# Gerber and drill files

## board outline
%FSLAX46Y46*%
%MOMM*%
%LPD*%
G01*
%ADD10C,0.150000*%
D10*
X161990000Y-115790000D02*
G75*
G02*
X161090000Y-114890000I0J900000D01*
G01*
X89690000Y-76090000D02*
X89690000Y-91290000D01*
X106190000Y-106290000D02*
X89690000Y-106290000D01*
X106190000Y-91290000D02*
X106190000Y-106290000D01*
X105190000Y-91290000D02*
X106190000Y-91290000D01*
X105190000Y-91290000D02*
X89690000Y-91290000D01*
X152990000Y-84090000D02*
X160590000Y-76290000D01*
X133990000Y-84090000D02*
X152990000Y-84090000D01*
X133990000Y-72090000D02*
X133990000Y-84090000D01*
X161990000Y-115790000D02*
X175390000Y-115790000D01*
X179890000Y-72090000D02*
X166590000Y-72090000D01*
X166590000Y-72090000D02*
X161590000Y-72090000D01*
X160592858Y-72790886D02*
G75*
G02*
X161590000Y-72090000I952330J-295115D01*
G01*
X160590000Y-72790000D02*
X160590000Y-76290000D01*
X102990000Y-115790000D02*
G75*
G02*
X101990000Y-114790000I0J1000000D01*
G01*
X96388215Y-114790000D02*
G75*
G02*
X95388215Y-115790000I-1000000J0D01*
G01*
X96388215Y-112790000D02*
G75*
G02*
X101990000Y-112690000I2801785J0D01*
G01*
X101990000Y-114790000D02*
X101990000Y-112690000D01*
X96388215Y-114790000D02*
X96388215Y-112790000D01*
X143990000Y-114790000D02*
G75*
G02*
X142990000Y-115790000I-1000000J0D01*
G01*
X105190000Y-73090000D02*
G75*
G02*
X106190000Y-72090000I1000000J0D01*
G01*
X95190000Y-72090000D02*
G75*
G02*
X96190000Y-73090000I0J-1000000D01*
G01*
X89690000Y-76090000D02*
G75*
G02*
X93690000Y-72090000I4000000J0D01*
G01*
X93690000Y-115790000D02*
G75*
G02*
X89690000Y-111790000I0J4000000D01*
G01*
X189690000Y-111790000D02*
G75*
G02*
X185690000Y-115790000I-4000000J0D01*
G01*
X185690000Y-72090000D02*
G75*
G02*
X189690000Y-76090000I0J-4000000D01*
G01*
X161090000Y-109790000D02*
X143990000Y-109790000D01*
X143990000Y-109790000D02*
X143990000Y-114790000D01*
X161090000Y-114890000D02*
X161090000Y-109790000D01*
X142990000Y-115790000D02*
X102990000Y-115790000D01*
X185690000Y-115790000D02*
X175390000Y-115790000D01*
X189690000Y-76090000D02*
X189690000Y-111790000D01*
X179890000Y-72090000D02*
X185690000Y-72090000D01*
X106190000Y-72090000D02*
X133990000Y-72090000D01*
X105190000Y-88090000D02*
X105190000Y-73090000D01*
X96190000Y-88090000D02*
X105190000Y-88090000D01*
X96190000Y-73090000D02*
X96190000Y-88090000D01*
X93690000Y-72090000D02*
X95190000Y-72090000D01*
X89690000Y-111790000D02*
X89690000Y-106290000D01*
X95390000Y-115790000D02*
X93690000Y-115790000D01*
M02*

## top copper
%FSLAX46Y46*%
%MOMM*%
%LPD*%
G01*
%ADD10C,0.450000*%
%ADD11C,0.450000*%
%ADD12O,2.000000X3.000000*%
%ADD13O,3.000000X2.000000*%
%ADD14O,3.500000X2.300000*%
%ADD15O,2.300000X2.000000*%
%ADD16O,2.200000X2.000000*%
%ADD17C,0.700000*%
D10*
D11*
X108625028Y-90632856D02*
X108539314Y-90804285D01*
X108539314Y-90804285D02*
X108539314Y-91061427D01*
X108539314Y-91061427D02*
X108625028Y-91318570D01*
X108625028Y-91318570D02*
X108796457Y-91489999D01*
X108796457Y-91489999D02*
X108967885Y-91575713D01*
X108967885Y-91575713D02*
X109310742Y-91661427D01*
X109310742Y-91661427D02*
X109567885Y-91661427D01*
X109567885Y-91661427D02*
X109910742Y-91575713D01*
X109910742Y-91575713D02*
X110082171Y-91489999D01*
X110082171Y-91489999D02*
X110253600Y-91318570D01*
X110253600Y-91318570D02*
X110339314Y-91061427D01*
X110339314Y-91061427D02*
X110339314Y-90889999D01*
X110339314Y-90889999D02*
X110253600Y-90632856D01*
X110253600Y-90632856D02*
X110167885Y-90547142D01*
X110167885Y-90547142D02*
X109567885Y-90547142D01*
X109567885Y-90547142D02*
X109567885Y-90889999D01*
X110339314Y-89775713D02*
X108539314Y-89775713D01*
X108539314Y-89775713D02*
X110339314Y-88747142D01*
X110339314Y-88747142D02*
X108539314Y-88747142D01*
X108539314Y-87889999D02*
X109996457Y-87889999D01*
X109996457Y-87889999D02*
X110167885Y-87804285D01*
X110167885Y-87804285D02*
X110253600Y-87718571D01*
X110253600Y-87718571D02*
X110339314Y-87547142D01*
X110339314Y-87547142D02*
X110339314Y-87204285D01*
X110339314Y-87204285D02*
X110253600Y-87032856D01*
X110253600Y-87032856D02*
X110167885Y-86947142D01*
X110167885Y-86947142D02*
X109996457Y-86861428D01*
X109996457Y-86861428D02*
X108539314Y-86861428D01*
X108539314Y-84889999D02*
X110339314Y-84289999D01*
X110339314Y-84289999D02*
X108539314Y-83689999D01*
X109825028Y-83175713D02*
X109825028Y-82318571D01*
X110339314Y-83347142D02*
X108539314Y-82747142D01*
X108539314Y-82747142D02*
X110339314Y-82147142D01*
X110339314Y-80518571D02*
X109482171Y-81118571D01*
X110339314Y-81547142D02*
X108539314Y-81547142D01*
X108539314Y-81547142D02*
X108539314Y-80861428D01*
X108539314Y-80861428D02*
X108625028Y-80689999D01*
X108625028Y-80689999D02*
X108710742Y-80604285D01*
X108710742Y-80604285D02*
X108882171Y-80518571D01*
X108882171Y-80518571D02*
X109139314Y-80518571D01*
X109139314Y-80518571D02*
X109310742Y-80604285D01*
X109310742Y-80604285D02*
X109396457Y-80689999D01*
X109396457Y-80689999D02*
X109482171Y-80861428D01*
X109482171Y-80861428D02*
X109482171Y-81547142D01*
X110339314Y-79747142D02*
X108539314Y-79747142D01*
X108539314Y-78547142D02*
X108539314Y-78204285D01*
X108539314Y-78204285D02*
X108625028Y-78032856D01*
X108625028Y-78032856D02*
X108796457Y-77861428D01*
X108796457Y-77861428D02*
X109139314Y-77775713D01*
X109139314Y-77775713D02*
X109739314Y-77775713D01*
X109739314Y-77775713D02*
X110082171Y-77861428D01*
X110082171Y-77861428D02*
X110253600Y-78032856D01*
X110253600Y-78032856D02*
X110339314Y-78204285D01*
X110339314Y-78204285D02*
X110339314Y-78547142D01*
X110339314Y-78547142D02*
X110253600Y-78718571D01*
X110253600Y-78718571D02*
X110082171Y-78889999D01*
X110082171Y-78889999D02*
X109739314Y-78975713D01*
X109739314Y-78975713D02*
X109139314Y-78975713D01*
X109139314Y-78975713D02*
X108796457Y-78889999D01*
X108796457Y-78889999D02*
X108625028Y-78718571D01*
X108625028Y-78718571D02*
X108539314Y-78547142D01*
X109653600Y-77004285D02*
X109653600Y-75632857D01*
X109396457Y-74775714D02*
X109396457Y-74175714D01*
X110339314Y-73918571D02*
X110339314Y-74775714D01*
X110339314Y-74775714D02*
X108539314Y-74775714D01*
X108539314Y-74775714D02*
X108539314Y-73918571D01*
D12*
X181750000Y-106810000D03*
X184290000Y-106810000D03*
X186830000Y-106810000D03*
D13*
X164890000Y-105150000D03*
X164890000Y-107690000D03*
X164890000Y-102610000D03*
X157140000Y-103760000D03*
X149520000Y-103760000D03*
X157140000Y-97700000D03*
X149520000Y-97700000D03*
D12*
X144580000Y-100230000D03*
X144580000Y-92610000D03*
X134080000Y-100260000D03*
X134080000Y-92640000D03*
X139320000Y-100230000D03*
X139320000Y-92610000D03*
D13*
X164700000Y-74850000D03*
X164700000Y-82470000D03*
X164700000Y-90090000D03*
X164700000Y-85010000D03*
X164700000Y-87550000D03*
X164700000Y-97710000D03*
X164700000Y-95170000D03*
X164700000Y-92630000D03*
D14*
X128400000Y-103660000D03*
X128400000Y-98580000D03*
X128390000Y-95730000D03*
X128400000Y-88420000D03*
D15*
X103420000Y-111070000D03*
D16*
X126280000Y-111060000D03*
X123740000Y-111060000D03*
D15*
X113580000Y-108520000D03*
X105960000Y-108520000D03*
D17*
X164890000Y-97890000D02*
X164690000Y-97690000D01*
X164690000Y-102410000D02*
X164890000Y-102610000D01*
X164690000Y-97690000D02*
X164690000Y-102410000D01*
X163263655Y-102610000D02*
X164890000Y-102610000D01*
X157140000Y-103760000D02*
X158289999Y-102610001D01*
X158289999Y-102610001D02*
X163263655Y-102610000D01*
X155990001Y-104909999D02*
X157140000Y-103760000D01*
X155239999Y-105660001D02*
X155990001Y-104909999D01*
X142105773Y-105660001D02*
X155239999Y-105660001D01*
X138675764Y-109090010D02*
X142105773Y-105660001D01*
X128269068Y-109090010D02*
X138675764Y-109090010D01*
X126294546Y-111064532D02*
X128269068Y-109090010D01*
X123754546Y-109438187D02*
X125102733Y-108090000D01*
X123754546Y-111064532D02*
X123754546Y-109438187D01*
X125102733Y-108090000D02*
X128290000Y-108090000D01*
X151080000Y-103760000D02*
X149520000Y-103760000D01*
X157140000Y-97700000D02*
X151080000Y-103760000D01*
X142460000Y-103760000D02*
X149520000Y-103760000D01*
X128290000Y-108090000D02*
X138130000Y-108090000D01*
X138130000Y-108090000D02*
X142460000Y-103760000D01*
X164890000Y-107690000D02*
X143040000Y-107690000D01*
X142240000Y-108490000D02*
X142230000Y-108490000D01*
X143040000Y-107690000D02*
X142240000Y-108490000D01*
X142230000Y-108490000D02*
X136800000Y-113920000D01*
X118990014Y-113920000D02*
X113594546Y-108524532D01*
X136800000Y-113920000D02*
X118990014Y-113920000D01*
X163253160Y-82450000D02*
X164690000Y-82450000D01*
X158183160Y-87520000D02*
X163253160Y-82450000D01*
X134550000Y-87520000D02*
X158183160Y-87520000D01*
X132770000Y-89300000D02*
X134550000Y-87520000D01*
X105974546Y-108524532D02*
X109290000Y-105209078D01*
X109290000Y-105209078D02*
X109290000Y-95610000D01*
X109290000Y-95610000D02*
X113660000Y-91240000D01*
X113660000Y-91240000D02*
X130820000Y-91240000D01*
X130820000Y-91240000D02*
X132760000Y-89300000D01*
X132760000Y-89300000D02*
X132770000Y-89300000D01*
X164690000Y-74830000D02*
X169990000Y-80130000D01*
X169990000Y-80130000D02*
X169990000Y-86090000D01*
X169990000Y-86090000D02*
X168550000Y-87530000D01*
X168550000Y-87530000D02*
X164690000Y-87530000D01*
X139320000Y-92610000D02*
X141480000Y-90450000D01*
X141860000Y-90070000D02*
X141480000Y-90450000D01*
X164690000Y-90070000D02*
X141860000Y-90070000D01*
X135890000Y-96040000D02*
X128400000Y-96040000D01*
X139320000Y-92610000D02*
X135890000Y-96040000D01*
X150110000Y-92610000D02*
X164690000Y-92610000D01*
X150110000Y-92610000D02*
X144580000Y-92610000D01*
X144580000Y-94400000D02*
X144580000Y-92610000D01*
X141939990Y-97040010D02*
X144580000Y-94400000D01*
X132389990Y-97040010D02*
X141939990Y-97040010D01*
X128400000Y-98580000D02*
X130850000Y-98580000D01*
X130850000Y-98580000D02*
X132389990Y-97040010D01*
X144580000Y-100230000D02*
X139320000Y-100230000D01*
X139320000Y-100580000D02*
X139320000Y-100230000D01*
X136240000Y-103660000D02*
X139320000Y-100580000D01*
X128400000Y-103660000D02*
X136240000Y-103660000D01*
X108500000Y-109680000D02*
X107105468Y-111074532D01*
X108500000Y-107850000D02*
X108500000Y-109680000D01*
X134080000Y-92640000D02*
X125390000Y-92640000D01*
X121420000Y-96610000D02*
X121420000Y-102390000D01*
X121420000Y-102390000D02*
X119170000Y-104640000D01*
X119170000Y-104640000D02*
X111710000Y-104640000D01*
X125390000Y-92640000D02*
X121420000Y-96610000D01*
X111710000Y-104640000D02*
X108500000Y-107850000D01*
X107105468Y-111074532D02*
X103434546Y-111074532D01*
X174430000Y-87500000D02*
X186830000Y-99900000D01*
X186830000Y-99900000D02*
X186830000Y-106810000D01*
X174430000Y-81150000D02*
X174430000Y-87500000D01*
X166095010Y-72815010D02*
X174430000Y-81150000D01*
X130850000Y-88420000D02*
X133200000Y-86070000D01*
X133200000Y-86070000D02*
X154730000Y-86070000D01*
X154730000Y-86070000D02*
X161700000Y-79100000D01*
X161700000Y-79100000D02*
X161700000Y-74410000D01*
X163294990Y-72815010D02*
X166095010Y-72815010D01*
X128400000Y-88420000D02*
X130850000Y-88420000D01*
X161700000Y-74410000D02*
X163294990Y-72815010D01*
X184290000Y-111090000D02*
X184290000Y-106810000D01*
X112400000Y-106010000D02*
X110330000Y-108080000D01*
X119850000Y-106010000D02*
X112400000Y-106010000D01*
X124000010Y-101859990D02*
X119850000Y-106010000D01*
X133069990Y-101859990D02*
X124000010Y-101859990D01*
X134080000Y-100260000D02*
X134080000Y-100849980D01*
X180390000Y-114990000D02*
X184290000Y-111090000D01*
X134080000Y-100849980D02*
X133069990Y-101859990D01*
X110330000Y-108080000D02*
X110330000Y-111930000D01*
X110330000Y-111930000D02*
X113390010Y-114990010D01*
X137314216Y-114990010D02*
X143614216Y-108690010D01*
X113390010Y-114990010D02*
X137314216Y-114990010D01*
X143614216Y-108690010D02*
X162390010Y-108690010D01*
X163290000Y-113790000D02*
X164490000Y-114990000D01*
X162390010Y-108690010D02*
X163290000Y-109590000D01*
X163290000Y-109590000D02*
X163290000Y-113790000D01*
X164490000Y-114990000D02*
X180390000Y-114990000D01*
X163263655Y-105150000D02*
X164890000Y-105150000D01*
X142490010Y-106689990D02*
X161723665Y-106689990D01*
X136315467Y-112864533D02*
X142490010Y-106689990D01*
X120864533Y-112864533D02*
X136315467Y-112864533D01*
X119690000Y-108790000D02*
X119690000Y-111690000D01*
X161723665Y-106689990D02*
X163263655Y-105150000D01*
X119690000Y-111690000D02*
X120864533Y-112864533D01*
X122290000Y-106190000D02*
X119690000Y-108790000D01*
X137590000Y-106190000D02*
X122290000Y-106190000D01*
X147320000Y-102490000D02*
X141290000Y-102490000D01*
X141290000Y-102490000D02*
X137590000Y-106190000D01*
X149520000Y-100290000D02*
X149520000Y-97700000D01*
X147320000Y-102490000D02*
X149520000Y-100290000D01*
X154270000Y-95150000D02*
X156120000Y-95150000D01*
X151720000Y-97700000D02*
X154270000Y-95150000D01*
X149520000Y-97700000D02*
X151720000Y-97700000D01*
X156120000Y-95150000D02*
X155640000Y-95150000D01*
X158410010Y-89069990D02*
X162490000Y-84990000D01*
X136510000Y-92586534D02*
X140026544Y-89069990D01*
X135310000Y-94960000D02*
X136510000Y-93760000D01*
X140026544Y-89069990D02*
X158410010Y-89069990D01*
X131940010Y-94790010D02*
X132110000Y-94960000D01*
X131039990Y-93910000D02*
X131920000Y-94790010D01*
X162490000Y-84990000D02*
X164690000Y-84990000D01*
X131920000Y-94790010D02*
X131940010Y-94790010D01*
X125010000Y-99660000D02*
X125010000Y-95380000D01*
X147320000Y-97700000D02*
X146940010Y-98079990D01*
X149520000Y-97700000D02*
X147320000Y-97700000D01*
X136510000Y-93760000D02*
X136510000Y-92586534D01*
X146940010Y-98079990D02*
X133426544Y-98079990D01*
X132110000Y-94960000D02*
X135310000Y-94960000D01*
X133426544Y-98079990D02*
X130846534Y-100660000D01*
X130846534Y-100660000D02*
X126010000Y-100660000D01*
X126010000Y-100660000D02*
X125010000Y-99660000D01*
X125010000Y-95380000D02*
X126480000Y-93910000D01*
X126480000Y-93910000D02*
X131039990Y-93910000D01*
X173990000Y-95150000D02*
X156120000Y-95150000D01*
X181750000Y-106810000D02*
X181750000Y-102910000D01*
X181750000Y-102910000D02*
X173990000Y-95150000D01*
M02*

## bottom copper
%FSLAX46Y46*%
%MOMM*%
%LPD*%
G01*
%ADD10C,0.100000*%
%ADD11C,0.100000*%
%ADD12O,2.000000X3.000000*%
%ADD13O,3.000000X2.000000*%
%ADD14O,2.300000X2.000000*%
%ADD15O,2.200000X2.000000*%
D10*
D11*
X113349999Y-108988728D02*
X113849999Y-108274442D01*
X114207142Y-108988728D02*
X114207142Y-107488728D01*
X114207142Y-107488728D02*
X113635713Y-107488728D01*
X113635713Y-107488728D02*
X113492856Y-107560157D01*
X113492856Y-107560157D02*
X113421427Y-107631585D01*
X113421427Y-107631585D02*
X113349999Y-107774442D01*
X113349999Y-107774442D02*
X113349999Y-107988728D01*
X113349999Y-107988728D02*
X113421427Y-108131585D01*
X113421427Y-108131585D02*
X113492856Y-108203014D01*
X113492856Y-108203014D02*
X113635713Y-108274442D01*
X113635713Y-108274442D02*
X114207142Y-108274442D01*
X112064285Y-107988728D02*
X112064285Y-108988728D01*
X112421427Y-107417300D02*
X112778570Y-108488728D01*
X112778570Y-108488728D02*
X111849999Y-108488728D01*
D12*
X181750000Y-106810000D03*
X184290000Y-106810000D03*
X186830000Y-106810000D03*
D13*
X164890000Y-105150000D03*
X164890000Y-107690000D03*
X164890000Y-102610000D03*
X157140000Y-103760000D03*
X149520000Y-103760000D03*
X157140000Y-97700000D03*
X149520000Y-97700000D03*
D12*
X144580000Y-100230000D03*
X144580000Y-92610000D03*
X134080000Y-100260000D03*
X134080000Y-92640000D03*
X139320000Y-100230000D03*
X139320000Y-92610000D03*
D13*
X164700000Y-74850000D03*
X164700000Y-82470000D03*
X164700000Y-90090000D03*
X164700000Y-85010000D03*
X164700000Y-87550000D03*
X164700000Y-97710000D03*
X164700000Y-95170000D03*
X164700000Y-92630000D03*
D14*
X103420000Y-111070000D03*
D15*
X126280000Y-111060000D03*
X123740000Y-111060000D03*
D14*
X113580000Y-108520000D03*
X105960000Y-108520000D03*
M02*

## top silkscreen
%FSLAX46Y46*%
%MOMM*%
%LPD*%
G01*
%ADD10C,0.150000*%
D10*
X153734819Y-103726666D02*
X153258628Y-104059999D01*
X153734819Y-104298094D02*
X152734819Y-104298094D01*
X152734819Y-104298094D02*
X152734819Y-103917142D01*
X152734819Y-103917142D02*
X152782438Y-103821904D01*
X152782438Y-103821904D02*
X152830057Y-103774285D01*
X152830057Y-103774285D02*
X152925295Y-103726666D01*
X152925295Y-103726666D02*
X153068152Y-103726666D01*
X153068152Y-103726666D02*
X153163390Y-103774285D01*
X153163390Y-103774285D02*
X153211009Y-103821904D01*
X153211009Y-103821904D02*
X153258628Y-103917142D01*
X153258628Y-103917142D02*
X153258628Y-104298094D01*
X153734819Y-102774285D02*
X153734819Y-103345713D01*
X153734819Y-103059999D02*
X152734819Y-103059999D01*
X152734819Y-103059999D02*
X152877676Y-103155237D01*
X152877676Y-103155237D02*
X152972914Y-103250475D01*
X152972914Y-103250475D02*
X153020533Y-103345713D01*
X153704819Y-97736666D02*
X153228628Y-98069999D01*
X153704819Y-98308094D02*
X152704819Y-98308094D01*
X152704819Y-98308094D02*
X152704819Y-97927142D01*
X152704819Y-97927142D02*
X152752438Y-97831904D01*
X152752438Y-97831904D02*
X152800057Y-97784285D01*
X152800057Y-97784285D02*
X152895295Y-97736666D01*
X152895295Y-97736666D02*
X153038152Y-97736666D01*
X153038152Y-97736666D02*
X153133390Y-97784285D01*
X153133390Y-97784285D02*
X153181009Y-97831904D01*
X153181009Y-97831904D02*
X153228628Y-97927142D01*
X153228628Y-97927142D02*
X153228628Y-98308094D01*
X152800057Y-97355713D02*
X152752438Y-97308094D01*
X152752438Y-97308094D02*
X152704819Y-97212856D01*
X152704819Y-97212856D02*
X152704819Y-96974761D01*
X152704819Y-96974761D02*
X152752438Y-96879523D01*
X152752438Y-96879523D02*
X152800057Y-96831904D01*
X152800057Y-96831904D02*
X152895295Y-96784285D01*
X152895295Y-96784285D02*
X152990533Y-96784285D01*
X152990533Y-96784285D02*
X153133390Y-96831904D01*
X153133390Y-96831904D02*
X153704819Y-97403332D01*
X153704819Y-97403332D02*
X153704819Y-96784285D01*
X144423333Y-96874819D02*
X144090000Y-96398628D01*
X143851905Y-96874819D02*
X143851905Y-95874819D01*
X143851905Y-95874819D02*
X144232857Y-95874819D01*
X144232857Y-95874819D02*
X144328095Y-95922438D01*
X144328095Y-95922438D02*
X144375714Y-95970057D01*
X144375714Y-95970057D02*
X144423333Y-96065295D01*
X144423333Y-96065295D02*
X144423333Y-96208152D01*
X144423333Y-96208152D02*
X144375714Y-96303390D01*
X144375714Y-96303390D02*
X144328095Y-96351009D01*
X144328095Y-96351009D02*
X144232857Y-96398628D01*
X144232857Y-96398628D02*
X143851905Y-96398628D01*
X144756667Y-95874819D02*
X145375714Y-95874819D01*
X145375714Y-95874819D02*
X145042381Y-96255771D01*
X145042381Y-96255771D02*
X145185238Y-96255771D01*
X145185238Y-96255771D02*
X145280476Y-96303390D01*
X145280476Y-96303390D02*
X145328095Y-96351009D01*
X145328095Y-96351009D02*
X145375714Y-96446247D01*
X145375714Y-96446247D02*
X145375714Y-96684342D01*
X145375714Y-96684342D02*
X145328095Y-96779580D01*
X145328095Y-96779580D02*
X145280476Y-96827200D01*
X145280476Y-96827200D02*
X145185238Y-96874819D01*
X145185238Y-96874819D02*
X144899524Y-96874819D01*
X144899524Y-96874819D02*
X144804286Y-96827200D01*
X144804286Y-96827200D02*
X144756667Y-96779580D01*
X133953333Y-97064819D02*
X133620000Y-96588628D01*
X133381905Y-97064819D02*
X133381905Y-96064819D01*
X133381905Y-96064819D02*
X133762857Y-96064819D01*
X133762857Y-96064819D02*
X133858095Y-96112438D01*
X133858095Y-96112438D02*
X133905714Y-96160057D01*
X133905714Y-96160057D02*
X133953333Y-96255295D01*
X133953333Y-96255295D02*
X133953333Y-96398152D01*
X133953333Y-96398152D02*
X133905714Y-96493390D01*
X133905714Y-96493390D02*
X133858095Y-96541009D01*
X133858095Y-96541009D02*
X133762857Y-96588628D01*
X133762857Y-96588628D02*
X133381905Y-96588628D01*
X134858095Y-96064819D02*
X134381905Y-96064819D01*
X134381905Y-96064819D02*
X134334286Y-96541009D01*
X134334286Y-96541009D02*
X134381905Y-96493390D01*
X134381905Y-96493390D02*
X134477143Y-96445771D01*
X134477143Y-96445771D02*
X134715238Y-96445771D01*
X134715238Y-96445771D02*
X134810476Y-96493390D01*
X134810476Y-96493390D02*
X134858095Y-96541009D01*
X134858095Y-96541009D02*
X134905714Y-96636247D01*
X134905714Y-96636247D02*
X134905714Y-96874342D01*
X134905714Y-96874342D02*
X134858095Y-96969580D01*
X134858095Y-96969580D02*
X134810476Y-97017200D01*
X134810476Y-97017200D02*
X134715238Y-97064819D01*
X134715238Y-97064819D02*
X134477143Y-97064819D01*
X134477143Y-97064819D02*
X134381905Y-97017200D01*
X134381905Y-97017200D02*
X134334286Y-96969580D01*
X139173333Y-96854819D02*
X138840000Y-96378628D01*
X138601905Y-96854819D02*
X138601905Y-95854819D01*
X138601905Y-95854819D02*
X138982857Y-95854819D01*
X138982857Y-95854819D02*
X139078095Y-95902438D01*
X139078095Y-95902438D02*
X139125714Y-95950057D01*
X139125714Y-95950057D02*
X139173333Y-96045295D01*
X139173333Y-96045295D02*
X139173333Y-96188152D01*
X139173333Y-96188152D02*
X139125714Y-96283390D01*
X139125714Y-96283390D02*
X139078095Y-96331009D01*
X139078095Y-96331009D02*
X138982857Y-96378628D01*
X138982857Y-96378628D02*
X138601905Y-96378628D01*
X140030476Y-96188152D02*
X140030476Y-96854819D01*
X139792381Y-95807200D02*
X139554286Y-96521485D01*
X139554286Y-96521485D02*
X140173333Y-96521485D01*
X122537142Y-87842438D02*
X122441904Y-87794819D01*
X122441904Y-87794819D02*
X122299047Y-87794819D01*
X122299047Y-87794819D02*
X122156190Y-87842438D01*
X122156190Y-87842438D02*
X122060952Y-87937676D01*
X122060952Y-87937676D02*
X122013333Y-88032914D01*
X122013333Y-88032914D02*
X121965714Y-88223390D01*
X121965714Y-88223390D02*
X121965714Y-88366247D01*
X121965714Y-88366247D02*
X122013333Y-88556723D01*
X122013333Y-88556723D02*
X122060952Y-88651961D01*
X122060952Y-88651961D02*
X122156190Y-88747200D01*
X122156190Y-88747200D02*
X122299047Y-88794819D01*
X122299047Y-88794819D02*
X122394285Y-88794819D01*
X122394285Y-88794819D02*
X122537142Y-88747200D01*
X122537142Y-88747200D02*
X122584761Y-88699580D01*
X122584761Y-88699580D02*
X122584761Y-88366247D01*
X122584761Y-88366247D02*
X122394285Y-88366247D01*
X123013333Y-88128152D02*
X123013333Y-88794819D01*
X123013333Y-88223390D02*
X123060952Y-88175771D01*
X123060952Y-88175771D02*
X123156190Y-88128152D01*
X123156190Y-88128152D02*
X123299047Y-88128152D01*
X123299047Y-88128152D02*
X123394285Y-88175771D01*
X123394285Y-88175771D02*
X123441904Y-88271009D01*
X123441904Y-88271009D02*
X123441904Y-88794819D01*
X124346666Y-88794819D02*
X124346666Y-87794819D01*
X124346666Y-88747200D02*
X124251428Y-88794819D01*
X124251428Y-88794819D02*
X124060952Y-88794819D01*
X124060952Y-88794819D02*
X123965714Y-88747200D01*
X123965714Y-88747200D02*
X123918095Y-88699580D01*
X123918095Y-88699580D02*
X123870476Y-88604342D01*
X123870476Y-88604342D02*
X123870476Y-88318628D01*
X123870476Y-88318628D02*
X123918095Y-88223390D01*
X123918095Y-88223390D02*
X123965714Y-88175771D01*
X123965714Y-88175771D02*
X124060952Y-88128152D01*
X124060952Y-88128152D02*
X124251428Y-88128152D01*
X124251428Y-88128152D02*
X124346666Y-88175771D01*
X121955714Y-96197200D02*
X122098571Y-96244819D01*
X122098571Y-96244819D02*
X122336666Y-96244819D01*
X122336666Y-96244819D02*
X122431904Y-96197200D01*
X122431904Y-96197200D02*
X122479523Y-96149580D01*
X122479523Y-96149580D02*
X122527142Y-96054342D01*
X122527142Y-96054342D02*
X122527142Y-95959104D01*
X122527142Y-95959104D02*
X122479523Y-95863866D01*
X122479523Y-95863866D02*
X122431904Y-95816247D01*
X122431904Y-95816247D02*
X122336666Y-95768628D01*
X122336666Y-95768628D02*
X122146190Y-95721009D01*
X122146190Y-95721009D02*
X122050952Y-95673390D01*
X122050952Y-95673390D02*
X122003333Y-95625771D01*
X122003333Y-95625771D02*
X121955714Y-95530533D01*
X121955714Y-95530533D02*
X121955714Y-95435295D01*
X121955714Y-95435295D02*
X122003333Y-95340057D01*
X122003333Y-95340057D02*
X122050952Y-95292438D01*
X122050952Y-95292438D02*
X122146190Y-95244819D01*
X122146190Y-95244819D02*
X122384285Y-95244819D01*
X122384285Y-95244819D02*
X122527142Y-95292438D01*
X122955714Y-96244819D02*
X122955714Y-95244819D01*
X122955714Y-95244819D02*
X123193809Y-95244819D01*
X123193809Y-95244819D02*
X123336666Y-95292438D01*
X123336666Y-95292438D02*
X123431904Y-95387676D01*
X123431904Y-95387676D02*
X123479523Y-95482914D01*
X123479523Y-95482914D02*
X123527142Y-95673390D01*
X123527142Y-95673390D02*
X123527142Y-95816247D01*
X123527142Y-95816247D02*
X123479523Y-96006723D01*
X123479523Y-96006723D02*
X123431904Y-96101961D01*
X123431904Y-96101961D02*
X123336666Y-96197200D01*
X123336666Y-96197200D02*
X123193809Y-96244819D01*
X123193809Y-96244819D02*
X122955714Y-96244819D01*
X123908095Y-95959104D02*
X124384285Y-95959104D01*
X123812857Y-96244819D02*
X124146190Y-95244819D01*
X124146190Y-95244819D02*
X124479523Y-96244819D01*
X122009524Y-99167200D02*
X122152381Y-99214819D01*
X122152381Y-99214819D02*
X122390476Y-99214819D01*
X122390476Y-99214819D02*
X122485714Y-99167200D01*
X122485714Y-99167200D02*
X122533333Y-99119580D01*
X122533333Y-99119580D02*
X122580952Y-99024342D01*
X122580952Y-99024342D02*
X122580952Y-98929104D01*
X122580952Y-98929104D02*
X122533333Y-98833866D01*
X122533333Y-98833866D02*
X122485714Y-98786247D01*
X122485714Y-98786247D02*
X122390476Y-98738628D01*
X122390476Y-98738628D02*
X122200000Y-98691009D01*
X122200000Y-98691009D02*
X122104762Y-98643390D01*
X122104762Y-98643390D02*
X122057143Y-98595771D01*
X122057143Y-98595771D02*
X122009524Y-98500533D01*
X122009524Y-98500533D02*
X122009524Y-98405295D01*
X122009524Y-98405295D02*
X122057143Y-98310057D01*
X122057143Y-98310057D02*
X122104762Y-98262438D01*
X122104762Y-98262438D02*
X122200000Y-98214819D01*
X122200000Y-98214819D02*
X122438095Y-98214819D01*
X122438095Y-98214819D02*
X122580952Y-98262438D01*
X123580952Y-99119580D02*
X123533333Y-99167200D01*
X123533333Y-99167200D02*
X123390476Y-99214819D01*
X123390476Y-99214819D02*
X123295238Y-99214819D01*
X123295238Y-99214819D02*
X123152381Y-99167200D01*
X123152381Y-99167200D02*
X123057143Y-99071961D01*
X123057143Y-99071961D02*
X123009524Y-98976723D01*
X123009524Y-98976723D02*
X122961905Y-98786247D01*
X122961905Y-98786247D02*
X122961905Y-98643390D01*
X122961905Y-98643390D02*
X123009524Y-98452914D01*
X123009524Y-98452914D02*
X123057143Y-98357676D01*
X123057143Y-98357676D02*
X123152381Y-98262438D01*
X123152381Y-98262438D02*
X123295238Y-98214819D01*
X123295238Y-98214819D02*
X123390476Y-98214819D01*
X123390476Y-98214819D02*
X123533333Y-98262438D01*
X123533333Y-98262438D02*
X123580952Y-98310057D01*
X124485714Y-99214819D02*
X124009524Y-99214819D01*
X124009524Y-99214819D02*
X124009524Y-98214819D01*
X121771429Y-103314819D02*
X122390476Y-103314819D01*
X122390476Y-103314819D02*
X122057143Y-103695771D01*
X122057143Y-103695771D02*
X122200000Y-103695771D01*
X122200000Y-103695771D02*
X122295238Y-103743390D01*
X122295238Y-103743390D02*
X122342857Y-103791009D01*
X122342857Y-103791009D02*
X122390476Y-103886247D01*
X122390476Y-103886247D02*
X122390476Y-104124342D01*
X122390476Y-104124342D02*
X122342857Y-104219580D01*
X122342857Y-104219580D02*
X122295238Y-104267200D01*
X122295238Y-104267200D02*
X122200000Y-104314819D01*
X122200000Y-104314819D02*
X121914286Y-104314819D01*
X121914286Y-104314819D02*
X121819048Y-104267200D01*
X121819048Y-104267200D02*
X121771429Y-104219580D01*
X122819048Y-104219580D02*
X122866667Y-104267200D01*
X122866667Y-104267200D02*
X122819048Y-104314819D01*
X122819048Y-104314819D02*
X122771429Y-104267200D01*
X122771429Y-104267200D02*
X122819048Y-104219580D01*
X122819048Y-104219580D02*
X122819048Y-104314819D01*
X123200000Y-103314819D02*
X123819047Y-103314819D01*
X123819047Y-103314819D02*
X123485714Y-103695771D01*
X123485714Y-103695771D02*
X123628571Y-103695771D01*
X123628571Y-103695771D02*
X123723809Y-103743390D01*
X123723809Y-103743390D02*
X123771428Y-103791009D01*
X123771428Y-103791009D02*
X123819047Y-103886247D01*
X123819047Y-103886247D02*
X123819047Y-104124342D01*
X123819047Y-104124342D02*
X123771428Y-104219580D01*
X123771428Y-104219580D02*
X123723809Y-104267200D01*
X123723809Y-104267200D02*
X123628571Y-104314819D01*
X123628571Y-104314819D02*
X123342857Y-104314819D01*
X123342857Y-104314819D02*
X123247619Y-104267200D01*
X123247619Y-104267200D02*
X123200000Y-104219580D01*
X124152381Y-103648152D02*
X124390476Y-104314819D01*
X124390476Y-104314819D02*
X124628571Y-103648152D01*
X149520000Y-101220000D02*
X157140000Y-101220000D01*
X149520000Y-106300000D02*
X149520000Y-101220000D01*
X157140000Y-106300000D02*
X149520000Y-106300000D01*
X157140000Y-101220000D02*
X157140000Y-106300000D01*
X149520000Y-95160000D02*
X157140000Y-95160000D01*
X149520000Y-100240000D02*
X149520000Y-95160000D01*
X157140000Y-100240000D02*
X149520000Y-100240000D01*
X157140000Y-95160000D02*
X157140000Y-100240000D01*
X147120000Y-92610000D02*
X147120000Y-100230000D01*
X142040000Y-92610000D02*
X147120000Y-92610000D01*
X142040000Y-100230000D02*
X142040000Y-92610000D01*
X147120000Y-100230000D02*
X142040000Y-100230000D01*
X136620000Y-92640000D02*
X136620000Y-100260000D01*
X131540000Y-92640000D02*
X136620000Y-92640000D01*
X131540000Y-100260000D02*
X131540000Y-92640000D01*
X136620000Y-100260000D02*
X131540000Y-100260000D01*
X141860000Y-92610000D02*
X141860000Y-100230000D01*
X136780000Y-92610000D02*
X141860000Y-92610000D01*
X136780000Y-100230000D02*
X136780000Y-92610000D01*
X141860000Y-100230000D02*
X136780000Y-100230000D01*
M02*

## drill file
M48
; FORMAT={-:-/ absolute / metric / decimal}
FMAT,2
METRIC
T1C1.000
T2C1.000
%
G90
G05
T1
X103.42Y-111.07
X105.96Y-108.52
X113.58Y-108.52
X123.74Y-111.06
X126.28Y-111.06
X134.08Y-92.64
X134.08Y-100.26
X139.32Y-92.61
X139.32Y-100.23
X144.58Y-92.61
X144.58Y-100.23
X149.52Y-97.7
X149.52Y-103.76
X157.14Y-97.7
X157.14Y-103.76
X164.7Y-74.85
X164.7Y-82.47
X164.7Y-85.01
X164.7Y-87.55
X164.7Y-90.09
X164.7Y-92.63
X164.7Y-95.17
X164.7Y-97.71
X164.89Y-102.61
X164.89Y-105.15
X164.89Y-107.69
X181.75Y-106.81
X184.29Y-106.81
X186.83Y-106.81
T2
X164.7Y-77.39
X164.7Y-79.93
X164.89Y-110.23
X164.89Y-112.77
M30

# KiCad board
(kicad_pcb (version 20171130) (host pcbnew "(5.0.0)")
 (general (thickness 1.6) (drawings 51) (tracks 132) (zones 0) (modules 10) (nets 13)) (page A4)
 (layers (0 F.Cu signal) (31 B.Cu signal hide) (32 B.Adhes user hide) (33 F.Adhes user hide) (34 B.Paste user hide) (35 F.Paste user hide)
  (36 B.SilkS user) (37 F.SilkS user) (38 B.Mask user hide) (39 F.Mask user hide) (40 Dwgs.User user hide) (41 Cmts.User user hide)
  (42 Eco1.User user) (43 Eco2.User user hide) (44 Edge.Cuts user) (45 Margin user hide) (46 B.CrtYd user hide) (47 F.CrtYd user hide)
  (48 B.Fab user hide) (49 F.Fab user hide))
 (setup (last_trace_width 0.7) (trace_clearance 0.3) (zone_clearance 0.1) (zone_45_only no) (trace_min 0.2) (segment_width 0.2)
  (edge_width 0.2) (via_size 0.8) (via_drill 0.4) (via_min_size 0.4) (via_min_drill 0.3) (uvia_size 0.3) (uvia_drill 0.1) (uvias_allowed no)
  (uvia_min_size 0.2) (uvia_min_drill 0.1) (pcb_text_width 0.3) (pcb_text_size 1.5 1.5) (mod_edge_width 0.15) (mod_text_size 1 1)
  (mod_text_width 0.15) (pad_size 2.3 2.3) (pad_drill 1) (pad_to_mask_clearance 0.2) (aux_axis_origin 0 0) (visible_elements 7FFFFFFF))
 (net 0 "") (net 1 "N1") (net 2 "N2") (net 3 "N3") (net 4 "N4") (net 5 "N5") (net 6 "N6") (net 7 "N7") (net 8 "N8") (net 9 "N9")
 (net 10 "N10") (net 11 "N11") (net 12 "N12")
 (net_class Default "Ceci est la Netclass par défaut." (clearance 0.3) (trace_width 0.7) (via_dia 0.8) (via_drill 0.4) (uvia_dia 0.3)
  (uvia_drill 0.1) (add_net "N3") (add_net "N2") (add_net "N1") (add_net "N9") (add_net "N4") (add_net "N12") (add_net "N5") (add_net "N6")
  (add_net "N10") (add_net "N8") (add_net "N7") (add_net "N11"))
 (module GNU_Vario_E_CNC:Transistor (layer F.Cu) (at 189.37 104.27 180)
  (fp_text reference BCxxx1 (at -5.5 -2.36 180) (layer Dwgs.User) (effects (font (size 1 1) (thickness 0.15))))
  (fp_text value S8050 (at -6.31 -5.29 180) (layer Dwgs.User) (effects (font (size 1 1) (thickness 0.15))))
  (pad 3 thru_hole oval (at 7.62 -2.54 180) (size 2 3) (drill 1) (layers *.Cu *.Mask) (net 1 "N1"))
  (pad 2 thru_hole oval (at 5.08 -2.54 180) (size 2 3) (drill 1) (layers *.Cu *.Mask) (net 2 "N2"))
  (pad 1 thru_hole oval (at 2.54 -2.54 180) (size 2 3) (drill 1) (layers *.Cu *.Mask) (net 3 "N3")))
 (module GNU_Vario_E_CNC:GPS (layer F.Cu) (at 164.89 102.61 270)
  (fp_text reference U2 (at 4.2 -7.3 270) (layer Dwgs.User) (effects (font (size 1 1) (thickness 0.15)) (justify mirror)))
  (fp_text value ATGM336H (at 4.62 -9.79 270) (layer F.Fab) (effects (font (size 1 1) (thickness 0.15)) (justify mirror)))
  (pad 2 thru_hole oval (at 2.54 0 270) (size 2 3) (drill 1) (layers *.Cu *.Mask) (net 1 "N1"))
  (pad 3 thru_hole oval (at 5.08 0 270) (size 2 3) (drill 1) (layers *.Cu *.Mask) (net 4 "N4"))
  (pad 1 thru_hole oval (at 0 0 270) (size 2 3) (drill 1) (layers *.Cu *.Mask) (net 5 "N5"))
  (pad "" np_thru_hole circle (at 7.62 0 270) (size 1 1) (drill 1) (layers *.Cu *.Mask))
  (pad "" np_thru_hole circle (at 10.16 0 270) (size 1 1) (drill 1) (layers *.Cu *.Mask)))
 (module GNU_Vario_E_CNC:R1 (layer F.Cu) (at 149.52 103.76 270)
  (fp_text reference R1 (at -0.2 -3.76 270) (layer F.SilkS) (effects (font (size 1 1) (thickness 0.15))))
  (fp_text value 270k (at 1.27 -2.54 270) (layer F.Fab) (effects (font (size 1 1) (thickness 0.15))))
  (fp_line (start -2.54 0) (end -2.54 -7.62) (layer F.SilkS) (width 0.15))
  (fp_line (start 2.54 0) (end -2.54 0) (layer F.SilkS) (width 0.15))
  (fp_line (start 2.54 -7.62) (end 2.54 0) (layer F.SilkS) (width 0.15))
  (fp_line (start -2.54 -7.62) (end 2.54 -7.62) (layer F.SilkS) (width 0.15))
  (pad 2 thru_hole oval (at 0 -7.62 270) (size 2 3) (drill 1) (layers *.Cu *.Mask) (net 5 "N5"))
  (pad 1 thru_hole oval (at 0 0 270) (size 2 3) (drill 1) (layers *.Cu *.Mask) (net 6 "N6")))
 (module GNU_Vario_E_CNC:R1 (layer F.Cu) (at 149.52 97.7 270)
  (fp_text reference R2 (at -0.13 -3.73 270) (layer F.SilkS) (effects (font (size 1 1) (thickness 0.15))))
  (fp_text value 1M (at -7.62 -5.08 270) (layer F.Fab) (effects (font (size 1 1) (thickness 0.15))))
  (fp_line (start -2.54 0) (end -2.54 -7.62) (layer F.SilkS) (width 0.15))
  (fp_line (start 2.54 0) (end -2.54 0) (layer F.SilkS) (width 0.15))
  (fp_line (start 2.54 -7.62) (end 2.54 0) (layer F.SilkS) (width 0.15))
  (fp_line (start -2.54 -7.62) (end 2.54 -7.62) (layer F.SilkS) (width 0.15))
  (pad 2 thru_hole oval (at 0 -7.62 270) (size 2 3) (drill 1) (layers *.Cu *.Mask) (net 6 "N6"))
  (pad 1 thru_hole oval (at 0 0 270) (size 2 3) (drill 1) (layers *.Cu *.Mask) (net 1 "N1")))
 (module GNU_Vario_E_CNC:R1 (layer F.Cu) (at 144.58 92.61 180)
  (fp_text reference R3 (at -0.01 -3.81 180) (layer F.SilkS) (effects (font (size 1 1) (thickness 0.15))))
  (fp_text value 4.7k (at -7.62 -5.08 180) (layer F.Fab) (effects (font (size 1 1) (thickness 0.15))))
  (fp_line (start -2.54 0) (end -2.54 -7.62) (layer F.SilkS) (width 0.15))
  (fp_line (start 2.54 0) (end -2.54 0) (layer F.SilkS) (width 0.15))
  (fp_line (start 2.54 -7.62) (end 2.54 0) (layer F.SilkS) (width 0.15))
  (fp_line (start -2.54 -7.62) (end 2.54 -7.62) (layer F.SilkS) (width 0.15))
  (pad 2 thru_hole oval (at 0 -7.62 180) (size 2 3) (drill 1) (layers *.Cu *.Mask) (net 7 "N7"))
  (pad 1 thru_hole oval (at 0 0 180) (size 2 3) (drill 1) (layers *.Cu *.Mask) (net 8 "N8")))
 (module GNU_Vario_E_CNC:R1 (layer F.Cu) (at 134.08 92.64 180)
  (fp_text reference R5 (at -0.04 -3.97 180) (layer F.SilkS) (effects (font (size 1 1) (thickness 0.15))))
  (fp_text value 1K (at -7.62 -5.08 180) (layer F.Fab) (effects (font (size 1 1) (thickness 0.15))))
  (fp_line (start -2.54 0) (end -2.54 -7.62) (layer F.SilkS) (width 0.15))
  (fp_line (start 2.54 0) (end -2.54 0) (layer F.SilkS) (width 0.15))
  (fp_line (start 2.54 -7.62) (end 2.54 0) (layer F.SilkS) (width 0.15))
  (fp_line (start -2.54 -7.62) (end 2.54 -7.62) (layer F.SilkS) (width 0.15))
  (pad 2 thru_hole oval (at 0 -7.62 180) (size 2 3) (drill 1) (layers *.Cu *.Mask) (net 2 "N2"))
  (pad 1 thru_hole oval (at 0 0 180) (size 2 3) (drill 1) (layers *.Cu *.Mask) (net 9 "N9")))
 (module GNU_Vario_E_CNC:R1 (layer F.Cu) (at 139.32 92.61 180)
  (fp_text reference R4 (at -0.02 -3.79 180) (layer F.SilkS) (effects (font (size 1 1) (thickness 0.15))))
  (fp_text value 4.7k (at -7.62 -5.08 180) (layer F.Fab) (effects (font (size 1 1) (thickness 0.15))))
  (fp_line (start -2.54 0) (end -2.54 -7.62) (layer F.SilkS) (width 0.15))
  (fp_line (start 2.54 0) (end -2.54 0) (layer F.SilkS) (width 0.15))
  (fp_line (start 2.54 -7.62) (end 2.54 0) (layer F.SilkS) (width 0.15))
  (fp_line (start -2.54 -7.62) (end 2.54 -7.62) (layer F.SilkS) (width 0.15))
  (pad 2 thru_hole oval (at 0 -7.62 180) (size 2 3) (drill 1) (layers *.Cu *.Mask) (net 7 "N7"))
  (pad 1 thru_hole oval (at 0 0 180) (size 2 3) (drill 1) (layers *.Cu *.Mask) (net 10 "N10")))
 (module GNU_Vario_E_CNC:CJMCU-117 (layer F.Cu) (at 167.24 87.55 90)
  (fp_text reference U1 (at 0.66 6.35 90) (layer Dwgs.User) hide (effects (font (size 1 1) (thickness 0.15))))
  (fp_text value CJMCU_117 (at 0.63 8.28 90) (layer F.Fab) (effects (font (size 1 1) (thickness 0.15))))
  (pad 10 thru_hole oval (at 12.7 -2.54 90) (size 2 3) (drill 1) (layers *.Cu *.Mask) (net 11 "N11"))
  (pad 7 thru_hole oval (at 5.08 -2.54 90) (size 2 3) (drill 1) (layers *.Cu *.Mask) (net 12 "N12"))
  (pad 4 thru_hole oval (at -2.54 -2.54 90) (size 2 3) (drill 1) (layers *.Cu *.Mask) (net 10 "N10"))
  (pad 6 thru_hole oval (at 2.54 -2.54 90) (size 2 3) (drill 1) (layers *.Cu *.Mask) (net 1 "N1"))
  (pad 5 thru_hole oval (at 0 -2.54 90) (size 2 3) (drill 1) (layers *.Cu *.Mask) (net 11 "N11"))
  (pad 1 thru_hole oval (at -10.16 -2.54 90) (size 2 3) (drill 1) (layers *.Cu *.Mask) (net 5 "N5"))
  (pad 2 thru_hole oval (at -7.62 -2.54 90) (size 2 3) (drill 1) (layers *.Cu *.Mask) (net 1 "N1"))
  (pad 3 thru_hole oval (at -5.08 -2.54 90) (size 2 3) (drill 1) (layers *.Cu *.Mask) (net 8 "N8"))
  (pad "" np_thru_hole circle (at 7.62 -2.54 90) (size 1 1) (drill 1) (layers *.Cu *.Mask))
  (pad "" np_thru_hole circle (at 10.16 -2.54 90) (size 1 1) (drill 1) (layers *.Cu *.Mask)))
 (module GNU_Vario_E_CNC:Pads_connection (layer F.Cu) (at 128.4 90.96)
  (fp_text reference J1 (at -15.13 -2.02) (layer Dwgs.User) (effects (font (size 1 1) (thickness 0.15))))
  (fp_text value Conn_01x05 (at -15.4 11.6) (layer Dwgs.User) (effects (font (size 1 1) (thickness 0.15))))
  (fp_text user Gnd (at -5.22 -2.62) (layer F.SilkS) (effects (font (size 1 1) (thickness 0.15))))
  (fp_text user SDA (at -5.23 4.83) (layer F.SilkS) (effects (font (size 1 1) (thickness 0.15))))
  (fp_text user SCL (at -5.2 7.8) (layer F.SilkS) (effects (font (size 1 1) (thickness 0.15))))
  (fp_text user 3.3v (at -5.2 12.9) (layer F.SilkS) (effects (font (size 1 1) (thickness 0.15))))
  (pad 5 smd oval (at 0 12.7) (size 3.5 2.3) (layers F.Cu F.Mask) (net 7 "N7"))
  (pad 4 smd oval (at 0 7.62) (size 3.5 2.3) (layers F.Cu F.Mask) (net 8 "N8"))
  (pad 3 smd oval (at -0.01 4.77) (size 3.5 2.3) (layers F.Cu F.Mask) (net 10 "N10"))
  (pad 1 smd oval (at 0 -2.54) (size 3.5 2.3) (layers F.Cu F.Mask) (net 3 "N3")))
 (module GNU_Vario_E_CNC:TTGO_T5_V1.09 (layer F.Cu) (at 131.91 108.74 90)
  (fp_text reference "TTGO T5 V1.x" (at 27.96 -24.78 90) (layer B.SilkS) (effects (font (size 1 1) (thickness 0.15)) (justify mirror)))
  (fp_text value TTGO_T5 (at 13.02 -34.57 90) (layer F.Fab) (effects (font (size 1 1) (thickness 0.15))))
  (pad 12 thru_hole oval (at -2.33 -28.49 90) (size 2 2.3) (drill 1) (layers *.Cu *.Mask) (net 9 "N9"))
  (pad 3 thru_hole oval (at -2.32 -5.63 90) (size 2 2.2) (drill 1) (layers *.Cu *.Mask) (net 5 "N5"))
  (pad 4 thru_hole oval (at -2.32 -8.17 90) (size 2 2.2) (drill 1) (layers *.Cu *.Mask) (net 6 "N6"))
  (pad 20 thru_hole oval (at 0.22 -18.33 90) (size 2 2.3) (drill 1) (layers *.Cu *.Mask) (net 4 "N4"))
  (pad 23 thru_hole oval (at 0.22 -25.95 90) (size 2 2.3) (drill 1) (layers *.Cu *.Mask) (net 12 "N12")))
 (gr_arc (start 161.99 114.89) (end 161.09 114.89) (angle -90) (layer Edge.Cuts) (width 0.15))
 (gr_line (start 89.69 76.09) (end 89.69 91.29) (layer Edge.Cuts) (width 0.15))
 (gr_line (start 106.19 106.29) (end 89.69 106.29) (layer Edge.Cuts) (width 0.15))
 (gr_line (start 106.19 91.29) (end 106.19 106.29) (layer Edge.Cuts) (width 0.15))
 (gr_line (start 105.19 91.29) (end 106.19 91.29) (layer Edge.Cuts) (width 0.15))
 (gr_line (start 105.19 91.29) (end 89.69 91.29) (layer Edge.Cuts) (width 0.15))
 (gr_line (start 152.99 84.09) (end 160.59 76.29) (layer Edge.Cuts) (width 0.15))
 (gr_line (start 133.99 84.09) (end 152.99 84.09) (layer Edge.Cuts) (width 0.15))
 (gr_line (start 133.99 72.09) (end 133.99 84.09) (layer Edge.Cuts) (width 0.15))
 (gr_line (start 161.99 115.79) (end 175.39 115.79) (layer Edge.Cuts) (width 0.15))
 (gr_line (start 179.89 72.09) (end 166.59 72.09) (layer Edge.Cuts) (width 0.15))
 (gr_line (start 166.59 72.09) (end 161.59 72.09) (layer Edge.Cuts) (width 0.15))
 (gr_arc (start 161.545188 73.086001) (end 161.59 72.09) (angle -75.35856355) (layer Edge.Cuts) (width 0.15))
 (gr_line (start 160.59 72.79) (end 160.59 76.29) (layer Edge.Cuts) (width 0.15))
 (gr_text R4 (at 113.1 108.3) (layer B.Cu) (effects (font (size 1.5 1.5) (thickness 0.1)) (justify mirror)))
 (gr_arc (start 102.99 114.79) (end 101.99 114.79) (angle -90) (layer Edge.Cuts) (width 0.15))
 (gr_arc (start 95.388215 114.79) (end 95.388215 115.79) (angle -90) (layer Edge.Cuts) (width 0.15))
 (gr_arc (start 99.19 112.79) (end 101.99 112.69) (angle -177.9545915) (layer Edge.Cuts) (width 0.15))
 (gr_line (start 101.99 114.79) (end 101.99 112.69) (layer Edge.Cuts) (width 0.15))
 (gr_line (start 96.388215 114.79) (end 96.388215 112.79) (layer Edge.Cuts) (width 0.15))
 (gr_arc (start 142.99 114.79) (end 142.99 115.79) (angle -90) (layer Edge.Cuts) (width 0.15))
 (gr_arc (start 106.19 73.09) (end 106.19 72.09) (angle -90) (layer Edge.Cuts) (width 0.15))
 (gr_arc (start 95.19 73.09) (end 96.19 73.09) (angle -90) (layer Edge.Cuts) (width 0.15))
 (gr_arc (start 93.69 76.09) (end 93.69 72.09) (angle -90) (layer Edge.Cuts) (width 0.15))
 (gr_arc (start 93.69 111.79) (end 89.69 111.79) (angle -90) (layer Edge.Cuts) (width 0.15))
 (gr_arc (start 185.69 111.79) (end 185.69 115.79) (angle -90) (layer Edge.Cuts) (width 0.15))
 (gr_arc (start 185.69 76.09) (end 189.69 76.09) (angle -90) (layer Edge.Cuts) (width 0.15))
 (gr_line (start 161.09 109.79) (end 143.99 109.79) (layer Edge.Cuts) (width 0.15))
 (gr_line (start 143.99 109.79) (end 143.99 114.79) (layer Edge.Cuts) (width 0.15))
 (gr_line (start 161.09 114.89) (end 161.09 109.79) (layer Edge.Cuts) (width 0.15))
 (gr_line (start 142.99 115.79) (end 102.99 115.79) (layer Edge.Cuts) (width 0.15))
 (gr_line (start 185.69 115.79) (end 175.39 115.79) (layer Edge.Cuts) (width 0.15))
 (gr_line (start 189.69 76.09) (end 189.69 111.79) (layer Edge.Cuts) (width 0.15))
 (gr_line (start 179.89 72.09) (end 185.69 72.09) (layer Edge.Cuts) (width 0.15))
 (gr_line (start 106.19 72.09) (end 133.99 72.09) (layer Edge.Cuts) (width 0.15))
 (gr_line (start 105.19 88.09) (end 105.19 73.09) (layer Edge.Cuts) (width 0.15))
 (gr_line (start 96.19 88.09) (end 105.19 88.09) (layer Edge.Cuts) (width 0.15))
 (gr_line (start 96.19 73.09) (end 96.19 88.09) (layer Edge.Cuts) (width 0.15))
 (gr_line (start 93.69 72.09) (end 95.19 72.09) (layer Edge.Cuts) (width 0.15))
 (gr_line (start 89.69 111.79) (end 89.69 106.29) (layer Edge.Cuts) (width 0.15))
 (gr_line (start 95.39 115.79) (end 93.69 115.79) (layer Edge.Cuts) (width 0.15))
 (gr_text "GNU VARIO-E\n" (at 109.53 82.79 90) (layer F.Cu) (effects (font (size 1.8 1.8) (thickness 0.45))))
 (segment (start 164.89 97.89) (end 164.69 97.69) (width 0.7) (layer F.Cu) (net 5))
 (segment (start 164.69 102.41) (end 164.89 102.61) (width 0.7) (layer F.Cu) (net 5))
 (segment (start 164.69 97.69) (end 164.69 102.41) (width 0.7) (layer F.Cu) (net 5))
 (segment (start 163.263655 102.61) (end 164.89 102.61) (width 0.7) (layer F.Cu) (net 5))
 (segment (start 157.14 103.76) (end 158.289999 102.610001) (width 0.7) (layer F.Cu) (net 5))
 (segment (start 158.289999 102.610001) (end 163.263655 102.61) (width 0.7) (layer F.Cu) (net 5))
 (segment (start 155.990001 104.909999) (end 157.14 103.76) (width 0.7) (layer F.Cu) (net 5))
 (segment (start 155.239999 105.660001) (end 155.990001 104.909999) (width 0.7) (layer F.Cu) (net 5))
 (segment (start 142.105773 105.660001) (end 155.239999 105.660001) (width 0.7) (layer F.Cu) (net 5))
 (segment (start 138.675764 109.09001) (end 142.105773 105.660001) (width 0.7) (layer F.Cu) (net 5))
 (segment (start 128.269068 109.09001) (end 138.675764 109.09001) (width 0.7) (layer F.Cu) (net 5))
 (segment (start 126.294546 111.064532) (end 128.269068 109.09001) (width 0.7) (layer F.Cu) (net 5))
 (segment (start 123.754546 109.438187) (end 125.102733 108.09) (width 0.7) (layer F.Cu) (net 6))
 (segment (start 123.754546 111.064532) (end 123.754546 109.438187) (width 0.7) (layer F.Cu) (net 6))
 (segment (start 125.102733 108.09) (end 128.29 108.09) (width 0.7) (layer F.Cu) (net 6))
 (segment (start 151.08 103.76) (end 149.52 103.76) (width 0.7) (layer F.Cu) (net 6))
 (segment (start 157.14 97.7) (end 151.08 103.76) (width 0.7) (layer F.Cu) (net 6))
 (segment (start 142.46 103.76) (end 149.52 103.76) (width 0.7) (layer F.Cu) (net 6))
 (segment (start 128.29 108.09) (end 138.13 108.09) (width 0.7) (layer F.Cu) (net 6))
 (segment (start 138.13 108.09) (end 142.46 103.76) (width 0.7) (layer F.Cu) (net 6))
 (segment (start 164.89 107.69) (end 143.04 107.69) (width 0.7) (layer F.Cu) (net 4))
 (segment (start 142.24 108.49) (end 142.23 108.49) (width 0.7) (layer F.Cu) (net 4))
 (segment (start 143.04 107.69) (end 142.24 108.49) (width 0.7) (layer F.Cu) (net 4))
 (segment (start 142.23 108.49) (end 136.8 113.92) (width 0.7) (layer F.Cu) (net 4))
 (segment (start 118.990014 113.92) (end 113.594546 108.524532) (width 0.7) (layer F.Cu) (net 4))
 (segment (start 136.8 113.92) (end 118.990014 113.92) (width 0.7) (layer F.Cu) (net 4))
 (segment (start 163.25316 82.45) (end 164.69 82.45) (width 0.7) (layer F.Cu) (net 12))
 (segment (start 158.18316 87.52) (end 163.25316 82.45) (width 0.7) (layer F.Cu) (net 12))
 (segment (start 134.55 87.52) (end 158.18316 87.52) (width 0.7) (layer F.Cu) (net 12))
 (segment (start 132.77 89.3) (end 134.55 87.52) (width 0.7) (layer F.Cu) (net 12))
 (segment (start 105.974546 108.524532) (end 109.29 105.209078) (width 0.7) (layer F.Cu) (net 12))
 (segment (start 109.29 105.209078) (end 109.29 95.61) (width 0.7) (layer F.Cu) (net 12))
 (segment (start 109.29 95.61) (end 113.66 91.24) (width 0.7) (layer F.Cu) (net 12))
 (segment (start 113.66 91.24) (end 130.82 91.24) (width 0.7) (layer F.Cu) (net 12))
 (segment (start 130.82 91.24) (end 132.76 89.3) (width 0.7) (layer F.Cu) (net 12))
 (segment (start 132.76 89.3) (end 132.77 89.3) (width 0.7) (layer F.Cu) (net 12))
 (segment (start 164.69 74.83) (end 169.99 80.13) (width 0.7) (layer F.Cu) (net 11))
 (segment (start 169.99 80.13) (end 169.99 86.09) (width 0.7) (layer F.Cu) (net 11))
 (segment (start 169.99 86.09) (end 168.55 87.53) (width 0.7) (layer F.Cu) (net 11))
 (segment (start 168.55 87.53) (end 164.69 87.53) (width 0.7) (layer F.Cu) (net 11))
 (segment (start 139.32 92.61) (end 141.48 90.45) (width 0.7) (layer F.Cu) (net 10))
 (segment (start 141.86 90.07) (end 141.48 90.45) (width 0.7) (layer F.Cu) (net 10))
 (segment (start 164.69 90.07) (end 141.86 90.07) (width 0.7) (layer F.Cu) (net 10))
 (segment (start 135.89 96.04) (end 128.4 96.04) (width 0.7) (layer F.Cu) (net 10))
 (segment (start 139.32 92.61) (end 135.89 96.04) (width 0.7) (layer F.Cu) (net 10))
 (segment (start 150.11 92.61) (end 164.69 92.61) (width 0.7) (layer F.Cu) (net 8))
 (segment (start 150.11 92.61) (end 144.58 92.61) (width 0.7) (layer F.Cu) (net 8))
 (segment (start 144.58 94.4) (end 144.58 92.61) (width 0.7) (layer F.Cu) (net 8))
 (segment (start 141.93999 97.04001) (end 144.58 94.4) (width 0.7) (layer F.Cu) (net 8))
 (segment (start 132.38999 97.04001) (end 141.93999 97.04001) (width 0.7) (layer F.Cu) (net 8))
 (segment (start 128.4 98.58) (end 130.85 98.58) (width 0.7) (layer F.Cu) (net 8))
 (segment (start 130.85 98.58) (end 132.38999 97.04001) (width 0.7) (layer F.Cu) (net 8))
 (segment (start 144.58 100.23) (end 139.32 100.23) (width 0.7) (layer F.Cu) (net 7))
 (segment (start 139.32 100.58) (end 139.32 100.23) (width 0.7) (layer F.Cu) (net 7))
 (segment (start 136.24 103.66) (end 139.32 100.58) (width 0.7) (layer F.Cu) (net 7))
 (segment (start 128.4 103.66) (end 136.24 103.66) (width 0.7) (layer F.Cu) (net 7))
 (segment (start 108.5 109.68) (end 107.105468 111.074532) (width 0.7) (layer F.Cu) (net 9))
 (segment (start 108.5 107.85) (end 108.5 109.68) (width 0.7) (layer F.Cu) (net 9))
 (segment (start 134.08 92.64) (end 125.39 92.64) (width 0.7) (layer F.Cu) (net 9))
 (segment (start 121.42 96.61) (end 121.42 102.39) (width 0.7) (layer F.Cu) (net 9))
 (segment (start 121.42 102.39) (end 119.17 104.64) (width 0.7) (layer F.Cu) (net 9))
 (segment (start 119.17 104.64) (end 111.71 104.64) (width 0.7) (layer F.Cu) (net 9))
 (segment (start 125.39 92.64) (end 121.42 96.61) (width 0.7) (layer F.Cu) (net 9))
 (segment (start 111.71 104.64) (end 108.5 107.85) (width 0.7) (layer F.Cu) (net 9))
 (segment (start 107.105468 111.074532) (end 103.434546 111.074532) (width 0.7) (layer F.Cu) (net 9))
 (segment (start 174.43 87.5) (end 186.83 99.9) (width 0.7) (layer F.Cu) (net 3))
 (segment (start 186.83 99.9) (end 186.83 106.81) (width 0.7) (layer F.Cu) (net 3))
 (segment (start 174.43 81.15) (end 174.43 87.5) (width 0.7) (layer F.Cu) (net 3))
 (segment (start 166.09501 72.81501) (end 174.43 81.15) (width 0.7) (layer F.Cu) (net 3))
 (segment (start 130.85 88.42) (end 133.2 86.07) (width 0.7) (layer F.Cu) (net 3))
 (segment (start 133.2 86.07) (end 154.73 86.07) (width 0.7) (layer F.Cu) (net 3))
 (segment (start 154.73 86.07) (end 161.7 79.1) (width 0.7) (layer F.Cu) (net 3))
 (segment (start 161.7 79.1) (end 161.7 74.41) (width 0.7) (layer F.Cu) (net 3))
 (segment (start 163.29499 72.81501) (end 166.09501 72.81501) (width 0.7) (layer F.Cu) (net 3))
 (segment (start 128.4 88.42) (end 130.85 88.42) (width 0.7) (layer F.Cu) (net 3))
 (segment (start 161.7 74.41) (end 163.29499 72.81501) (width 0.7) (layer F.Cu) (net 3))
 (segment (start 184.29 111.09) (end 184.29 106.81) (width 0.7) (layer F.Cu) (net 2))
 (segment (start 112.4 106.01) (end 110.33 108.08) (width 0.7) (layer F.Cu) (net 2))
 (segment (start 119.85 106.01) (end 112.4 106.01) (width 0.7) (layer F.Cu) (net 2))
 (segment (start 124.00001 101.85999) (end 119.85 106.01) (width 0.7) (layer F.Cu) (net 2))
 (segment (start 133.06999 101.85999) (end 124.00001 101.85999) (width 0.7) (layer F.Cu) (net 2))
 (segment (start 134.08 100.26) (end 134.08 100.84998) (width 0.7) (layer F.Cu) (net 2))
 (segment (start 180.39 114.99) (end 184.29 111.09) (width 0.7) (layer F.Cu) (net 2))
 (segment (start 134.08 100.84998) (end 133.06999 101.85999) (width 0.7) (layer F.Cu) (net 2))
 (segment (start 110.33 108.08) (end 110.33 111.93) (width 0.7) (layer F.Cu) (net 2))
 (segment (start 110.33 111.93) (end 113.39001 114.99001) (width 0.7) (layer F.Cu) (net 2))
 (segment (start 137.314216 114.99001) (end 143.614216 108.69001) (width 0.7) (layer F.Cu) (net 2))
 (segment (start 113.39001 114.99001) (end 137.314216 114.99001) (width 0.7) (layer F.Cu) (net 2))
 (segment (start 143.614216 108.69001) (end 162.39001 108.69001) (width 0.7) (layer F.Cu) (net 2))
 (segment (start 163.29 113.79) (end 164.49 114.99) (width 0.7) (layer F.Cu) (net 2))
 (segment (start 162.39001 108.69001) (end 163.29 109.59) (width 0.7) (layer F.Cu) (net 2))
 (segment (start 163.29 109.59) (end 163.29 113.79) (width 0.7) (layer F.Cu) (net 2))
 (segment (start 164.49 114.99) (end 180.39 114.99) (width 0.7) (layer F.Cu) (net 2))
 (segment (start 163.263655 105.15) (end 164.89 105.15) (width 0.7) (layer F.Cu) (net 1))
 (segment (start 142.49001 106.68999) (end 161.723665 106.68999) (width 0.7) (layer F.Cu) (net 1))
 (segment (start 136.315467 112.864533) (end 142.49001 106.68999) (width 0.7) (layer F.Cu) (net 1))
 (segment (start 120.864533 112.864533) (end 136.315467 112.864533) (width 0.7) (layer F.Cu) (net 1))
 (segment (start 119.69 108.79) (end 119.69 111.69) (width 0.7) (layer F.Cu) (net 1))
 (segment (start 161.723665 106.68999) (end 163.263655 105.15) (width 0.7) (layer F.Cu) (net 1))
 (segment (start 119.69 111.69) (end 120.864533 112.864533) (width 0.7) (layer F.Cu) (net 1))
 (segment (start 122.29 106.19) (end 119.69 108.79) (width 0.7) (layer F.Cu) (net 1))
 (segment (start 137.59 106.19) (end 122.29 106.19) (width 0.7) (layer F.Cu) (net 1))
 (segment (start 147.32 102.49) (end 141.29 102.49) (width 0.7) (layer F.Cu) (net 1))
 (segment (start 141.29 102.49) (end 137.59 106.19) (width 0.7) (layer F.Cu) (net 1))
 (segment (start 149.52 100.29) (end 149.52 97.7) (width 0.7) (layer F.Cu) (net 1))
 (segment (start 147.32 102.49) (end 149.52 100.29) (width 0.7) (layer F.Cu) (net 1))
 (segment (start 154.27 95.15) (end 156.12 95.15) (width 0.7) (layer F.Cu) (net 1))
 (segment (start 151.72 97.7) (end 154.27 95.15) (width 0.7) (layer F.Cu) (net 1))
 (segment (start 149.52 97.7) (end 151.72 97.7) (width 0.7) (layer F.Cu) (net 1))
 (segment (start 156.12 95.15) (end 155.64 95.15) (width 0.7) (layer F.Cu) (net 1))
 (segment (start 158.41001 89.06999) (end 162.49 84.99) (width 0.7) (layer F.Cu) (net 1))
 (segment (start 136.51 92.586534) (end 140.026544 89.06999) (width 0.7) (layer F.Cu) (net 1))
 (segment (start 135.31 94.96) (end 136.51 93.76) (width 0.7) (layer F.Cu) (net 1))
 (segment (start 140.026544 89.06999) (end 158.41001 89.06999) (width 0.7) (layer F.Cu) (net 1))
 (segment (start 131.94001 94.79001) (end 132.11 94.96) (width 0.7) (layer F.Cu) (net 1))
 (segment (start 131.03999 93.91) (end 131.92 94.79001) (width 0.7) (layer F.Cu) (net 1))
 (segment (start 162.49 84.99) (end 164.69 84.99) (width 0.7) (layer F.Cu) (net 1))
 (segment (start 131.92 94.79001) (end 131.94001 94.79001) (width 0.7) (layer F.Cu) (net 1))
 (segment (start 125.01 99.66) (end 125.01 95.38) (width 0.7) (layer F.Cu) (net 1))
 (segment (start 147.32 97.7) (end 146.94001 98.07999) (width 0.7) (layer F.Cu) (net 1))
 (segment (start 149.52 97.7) (end 147.32 97.7) (width 0.7) (layer F.Cu) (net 1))
 (segment (start 136.51 93.76) (end 136.51 92.586534) (width 0.7) (layer F.Cu) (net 1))
 (segment (start 146.94001 98.07999) (end 133.426544 98.07999) (width 0.7) (layer F.Cu) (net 1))
 (segment (start 132.11 94.96) (end 135.31 94.96) (width 0.7) (layer F.Cu) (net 1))
 (segment (start 133.426544 98.07999) (end 130.846534 100.66) (width 0.7) (layer F.Cu) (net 1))
 (segment (start 130.846534 100.66) (end 126.01 100.66) (width 0.7) (layer F.Cu) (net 1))
 (segment (start 126.01 100.66) (end 125.01 99.66) (width 0.7) (layer F.Cu) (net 1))
 (segment (start 125.01 95.38) (end 126.48 93.91) (width 0.7) (layer F.Cu) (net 1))
 (segment (start 126.48 93.91) (end 131.03999 93.91) (width 0.7) (layer F.Cu) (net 1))
 (segment (start 173.99 95.15) (end 156.12 95.15) (width 0.7) (layer F.Cu) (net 1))
 (segment (start 181.75 106.81) (end 181.75 102.91) (width 0.7) (layer F.Cu) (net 1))
 (segment (start 181.75 102.91) (end 173.99 95.15) (width 0.7) (layer F.Cu) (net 1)))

